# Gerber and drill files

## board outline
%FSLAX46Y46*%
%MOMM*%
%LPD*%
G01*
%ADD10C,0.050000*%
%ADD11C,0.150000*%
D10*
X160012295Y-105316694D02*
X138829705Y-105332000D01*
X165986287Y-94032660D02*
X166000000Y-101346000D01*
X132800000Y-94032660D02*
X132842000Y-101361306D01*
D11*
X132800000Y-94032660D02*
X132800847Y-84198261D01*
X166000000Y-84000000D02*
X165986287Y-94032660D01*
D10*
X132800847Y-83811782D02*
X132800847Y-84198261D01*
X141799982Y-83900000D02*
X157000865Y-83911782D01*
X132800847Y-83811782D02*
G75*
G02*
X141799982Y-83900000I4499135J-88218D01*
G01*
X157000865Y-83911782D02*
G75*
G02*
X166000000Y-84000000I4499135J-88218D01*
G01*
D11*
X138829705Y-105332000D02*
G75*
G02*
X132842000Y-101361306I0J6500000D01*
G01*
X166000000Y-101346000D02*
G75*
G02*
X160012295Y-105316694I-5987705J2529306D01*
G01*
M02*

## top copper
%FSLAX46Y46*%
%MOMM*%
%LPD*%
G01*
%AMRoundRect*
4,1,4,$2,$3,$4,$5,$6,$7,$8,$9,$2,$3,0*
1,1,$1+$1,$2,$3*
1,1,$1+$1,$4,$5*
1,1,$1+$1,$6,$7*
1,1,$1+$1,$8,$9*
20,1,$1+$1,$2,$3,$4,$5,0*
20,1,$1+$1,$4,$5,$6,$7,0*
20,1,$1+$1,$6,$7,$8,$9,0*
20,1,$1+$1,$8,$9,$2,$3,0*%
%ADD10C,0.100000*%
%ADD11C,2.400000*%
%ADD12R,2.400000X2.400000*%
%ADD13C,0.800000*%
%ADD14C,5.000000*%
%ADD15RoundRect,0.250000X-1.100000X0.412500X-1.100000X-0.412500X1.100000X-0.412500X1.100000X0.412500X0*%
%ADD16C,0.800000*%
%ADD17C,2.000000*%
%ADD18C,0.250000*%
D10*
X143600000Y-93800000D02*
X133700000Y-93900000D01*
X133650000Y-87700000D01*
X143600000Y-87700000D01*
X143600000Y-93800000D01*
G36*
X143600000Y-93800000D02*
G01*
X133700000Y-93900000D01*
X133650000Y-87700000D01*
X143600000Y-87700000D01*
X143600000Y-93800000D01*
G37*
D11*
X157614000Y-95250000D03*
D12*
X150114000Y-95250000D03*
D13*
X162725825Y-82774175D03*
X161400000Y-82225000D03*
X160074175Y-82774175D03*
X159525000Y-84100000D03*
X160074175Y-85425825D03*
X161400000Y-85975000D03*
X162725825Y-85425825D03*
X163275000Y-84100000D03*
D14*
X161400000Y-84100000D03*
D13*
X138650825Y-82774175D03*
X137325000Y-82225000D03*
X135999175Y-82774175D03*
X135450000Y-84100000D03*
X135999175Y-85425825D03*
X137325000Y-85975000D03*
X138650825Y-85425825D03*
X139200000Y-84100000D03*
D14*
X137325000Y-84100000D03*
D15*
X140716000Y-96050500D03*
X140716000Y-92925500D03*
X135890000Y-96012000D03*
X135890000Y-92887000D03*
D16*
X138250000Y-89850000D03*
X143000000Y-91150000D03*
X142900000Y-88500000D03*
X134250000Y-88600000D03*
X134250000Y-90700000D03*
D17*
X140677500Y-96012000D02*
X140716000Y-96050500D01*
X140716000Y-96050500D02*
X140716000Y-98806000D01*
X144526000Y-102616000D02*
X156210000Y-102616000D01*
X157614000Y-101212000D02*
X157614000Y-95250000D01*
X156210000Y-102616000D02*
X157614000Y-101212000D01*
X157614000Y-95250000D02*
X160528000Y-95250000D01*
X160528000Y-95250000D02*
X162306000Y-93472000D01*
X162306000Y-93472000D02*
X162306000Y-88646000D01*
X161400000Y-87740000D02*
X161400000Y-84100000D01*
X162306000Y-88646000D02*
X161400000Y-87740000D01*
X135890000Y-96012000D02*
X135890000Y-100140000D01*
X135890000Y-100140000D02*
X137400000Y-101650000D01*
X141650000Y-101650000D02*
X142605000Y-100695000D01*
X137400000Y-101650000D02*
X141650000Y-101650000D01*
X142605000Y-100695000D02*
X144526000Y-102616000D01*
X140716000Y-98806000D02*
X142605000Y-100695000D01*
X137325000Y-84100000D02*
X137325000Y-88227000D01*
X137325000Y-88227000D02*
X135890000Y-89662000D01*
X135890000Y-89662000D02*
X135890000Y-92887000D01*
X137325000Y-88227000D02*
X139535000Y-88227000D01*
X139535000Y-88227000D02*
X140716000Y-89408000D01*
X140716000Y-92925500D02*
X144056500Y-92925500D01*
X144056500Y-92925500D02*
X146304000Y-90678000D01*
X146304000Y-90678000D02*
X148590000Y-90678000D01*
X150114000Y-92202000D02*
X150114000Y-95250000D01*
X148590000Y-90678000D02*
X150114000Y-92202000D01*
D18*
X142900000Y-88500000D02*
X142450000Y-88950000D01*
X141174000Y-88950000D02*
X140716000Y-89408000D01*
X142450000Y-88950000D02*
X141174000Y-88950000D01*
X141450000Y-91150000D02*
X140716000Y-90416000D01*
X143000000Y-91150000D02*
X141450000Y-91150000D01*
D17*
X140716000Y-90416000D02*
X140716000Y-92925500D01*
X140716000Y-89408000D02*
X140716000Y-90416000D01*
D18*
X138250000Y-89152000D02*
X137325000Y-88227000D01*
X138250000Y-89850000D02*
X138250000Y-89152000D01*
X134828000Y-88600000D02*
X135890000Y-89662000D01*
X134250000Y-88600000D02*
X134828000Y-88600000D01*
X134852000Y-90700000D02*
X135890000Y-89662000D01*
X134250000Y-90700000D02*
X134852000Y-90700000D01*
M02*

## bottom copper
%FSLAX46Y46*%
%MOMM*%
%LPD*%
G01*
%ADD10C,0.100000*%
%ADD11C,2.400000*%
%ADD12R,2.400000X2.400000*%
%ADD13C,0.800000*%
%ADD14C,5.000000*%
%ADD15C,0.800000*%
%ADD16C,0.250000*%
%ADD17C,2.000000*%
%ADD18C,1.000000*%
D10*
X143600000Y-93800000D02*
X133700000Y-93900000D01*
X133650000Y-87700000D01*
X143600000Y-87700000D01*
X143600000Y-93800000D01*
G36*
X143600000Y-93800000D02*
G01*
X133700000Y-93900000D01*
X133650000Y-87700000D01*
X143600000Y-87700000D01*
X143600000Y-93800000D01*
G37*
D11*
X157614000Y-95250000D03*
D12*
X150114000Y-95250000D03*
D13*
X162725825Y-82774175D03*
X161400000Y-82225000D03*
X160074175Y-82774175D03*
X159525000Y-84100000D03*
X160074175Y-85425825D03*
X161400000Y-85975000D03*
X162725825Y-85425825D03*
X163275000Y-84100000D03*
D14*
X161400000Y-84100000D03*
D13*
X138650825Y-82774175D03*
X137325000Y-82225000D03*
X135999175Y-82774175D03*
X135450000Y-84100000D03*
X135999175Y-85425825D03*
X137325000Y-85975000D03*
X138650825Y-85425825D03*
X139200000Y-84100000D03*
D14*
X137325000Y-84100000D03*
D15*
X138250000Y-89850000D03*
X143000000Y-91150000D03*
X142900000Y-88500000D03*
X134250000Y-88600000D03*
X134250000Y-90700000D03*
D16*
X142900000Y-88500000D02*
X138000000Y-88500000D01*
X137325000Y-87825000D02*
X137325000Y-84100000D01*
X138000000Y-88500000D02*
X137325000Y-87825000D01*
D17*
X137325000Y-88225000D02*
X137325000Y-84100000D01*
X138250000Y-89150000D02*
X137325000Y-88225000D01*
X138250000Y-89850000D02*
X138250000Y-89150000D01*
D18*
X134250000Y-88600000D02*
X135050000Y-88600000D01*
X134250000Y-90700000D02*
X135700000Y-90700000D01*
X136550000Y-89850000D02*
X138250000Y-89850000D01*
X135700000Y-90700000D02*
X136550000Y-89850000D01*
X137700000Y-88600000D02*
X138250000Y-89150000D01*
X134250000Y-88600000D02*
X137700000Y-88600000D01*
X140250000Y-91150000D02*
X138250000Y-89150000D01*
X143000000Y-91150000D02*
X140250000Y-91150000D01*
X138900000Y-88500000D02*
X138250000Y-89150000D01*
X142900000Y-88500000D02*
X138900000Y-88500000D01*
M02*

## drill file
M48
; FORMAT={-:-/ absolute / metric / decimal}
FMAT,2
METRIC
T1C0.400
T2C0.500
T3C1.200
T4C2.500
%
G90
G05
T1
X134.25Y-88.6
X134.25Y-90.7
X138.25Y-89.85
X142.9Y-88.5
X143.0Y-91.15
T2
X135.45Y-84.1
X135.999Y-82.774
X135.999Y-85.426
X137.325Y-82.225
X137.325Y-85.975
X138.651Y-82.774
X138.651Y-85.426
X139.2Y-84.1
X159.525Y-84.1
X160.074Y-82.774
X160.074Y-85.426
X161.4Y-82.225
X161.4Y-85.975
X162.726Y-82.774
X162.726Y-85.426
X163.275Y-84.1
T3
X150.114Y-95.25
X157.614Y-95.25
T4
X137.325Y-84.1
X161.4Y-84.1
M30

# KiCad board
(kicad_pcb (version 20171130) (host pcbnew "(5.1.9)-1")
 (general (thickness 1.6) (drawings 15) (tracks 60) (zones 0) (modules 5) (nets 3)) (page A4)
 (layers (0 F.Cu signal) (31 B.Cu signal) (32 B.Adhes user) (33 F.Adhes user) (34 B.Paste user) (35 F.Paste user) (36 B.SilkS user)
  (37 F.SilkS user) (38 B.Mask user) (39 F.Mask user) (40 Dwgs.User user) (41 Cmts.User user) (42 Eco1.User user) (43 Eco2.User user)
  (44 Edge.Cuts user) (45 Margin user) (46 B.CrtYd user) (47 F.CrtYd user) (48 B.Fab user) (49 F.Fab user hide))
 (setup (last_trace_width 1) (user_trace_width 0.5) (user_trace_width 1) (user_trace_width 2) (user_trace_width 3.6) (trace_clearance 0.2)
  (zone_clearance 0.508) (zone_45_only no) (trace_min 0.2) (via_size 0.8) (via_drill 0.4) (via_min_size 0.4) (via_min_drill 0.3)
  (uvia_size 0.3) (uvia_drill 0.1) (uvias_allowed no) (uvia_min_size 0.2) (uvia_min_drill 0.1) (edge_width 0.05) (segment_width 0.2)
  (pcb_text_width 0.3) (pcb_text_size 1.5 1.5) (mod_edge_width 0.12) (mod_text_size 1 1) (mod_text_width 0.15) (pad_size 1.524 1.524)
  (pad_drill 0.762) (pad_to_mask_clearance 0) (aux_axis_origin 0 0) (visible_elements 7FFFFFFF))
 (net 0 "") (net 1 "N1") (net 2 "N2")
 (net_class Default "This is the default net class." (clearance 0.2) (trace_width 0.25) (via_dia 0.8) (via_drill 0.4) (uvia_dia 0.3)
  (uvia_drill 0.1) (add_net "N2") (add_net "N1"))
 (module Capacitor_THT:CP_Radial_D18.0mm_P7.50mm (layer F.Cu) (at 150.114 95.25)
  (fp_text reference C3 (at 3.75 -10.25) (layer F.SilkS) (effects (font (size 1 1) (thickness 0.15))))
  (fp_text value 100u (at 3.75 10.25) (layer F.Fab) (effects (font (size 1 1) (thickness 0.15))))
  (pad 2 thru_hole circle (at 7.5 0) (size 2.4 2.4) (drill 1.2) (layers *.Cu *.Mask) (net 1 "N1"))
  (pad 1 thru_hole rect (at 0 0) (size 2.4 2.4) (drill 1.2) (layers *.Cu *.Mask) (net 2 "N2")))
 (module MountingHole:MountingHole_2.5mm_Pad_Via (layer F.Cu) (at 161.4 84.1)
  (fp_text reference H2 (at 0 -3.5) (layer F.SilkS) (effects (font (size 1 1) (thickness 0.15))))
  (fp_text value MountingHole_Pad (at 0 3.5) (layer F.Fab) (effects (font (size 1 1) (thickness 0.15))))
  (pad 1 thru_hole circle (at 1.325825 -1.325825) (size 0.8 0.8) (drill 0.5) (layers *.Cu *.Mask) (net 1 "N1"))
  (pad 1 thru_hole circle (at 0 -1.875) (size 0.8 0.8) (drill 0.5) (layers *.Cu *.Mask) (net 1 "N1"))
  (pad 1 thru_hole circle (at -1.325825 -1.325825) (size 0.8 0.8) (drill 0.5) (layers *.Cu *.Mask) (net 1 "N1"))
  (pad 1 thru_hole circle (at -1.875 0) (size 0.8 0.8) (drill 0.5) (layers *.Cu *.Mask) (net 1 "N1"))
  (pad 1 thru_hole circle (at -1.325825 1.325825) (size 0.8 0.8) (drill 0.5) (layers *.Cu *.Mask) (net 1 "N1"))
  (pad 1 thru_hole circle (at 0 1.875) (size 0.8 0.8) (drill 0.5) (layers *.Cu *.Mask) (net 1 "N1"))
  (pad 1 thru_hole circle (at 1.325825 1.325825) (size 0.8 0.8) (drill 0.5) (layers *.Cu *.Mask) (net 1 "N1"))
  (pad 1 thru_hole circle (at 1.875 0) (size 0.8 0.8) (drill 0.5) (layers *.Cu *.Mask) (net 1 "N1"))
  (pad 1 thru_hole circle (at 0 0) (size 5 5) (drill 2.5) (layers *.Cu *.Mask) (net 1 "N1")))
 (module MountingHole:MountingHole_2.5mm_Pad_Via (layer F.Cu) (at 137.325 84.1)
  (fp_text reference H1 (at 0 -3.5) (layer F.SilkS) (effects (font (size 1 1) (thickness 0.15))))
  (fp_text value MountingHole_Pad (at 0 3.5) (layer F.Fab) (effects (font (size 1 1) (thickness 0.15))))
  (pad 1 thru_hole circle (at 1.325825 -1.325825) (size 0.8 0.8) (drill 0.5) (layers *.Cu *.Mask) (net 2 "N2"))
  (pad 1 thru_hole circle (at 0 -1.875) (size 0.8 0.8) (drill 0.5) (layers *.Cu *.Mask) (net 2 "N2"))
  (pad 1 thru_hole circle (at -1.325825 -1.325825) (size 0.8 0.8) (drill 0.5) (layers *.Cu *.Mask) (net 2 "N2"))
  (pad 1 thru_hole circle (at -1.875 0) (size 0.8 0.8) (drill 0.5) (layers *.Cu *.Mask) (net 2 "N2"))
  (pad 1 thru_hole circle (at -1.325825 1.325825) (size 0.8 0.8) (drill 0.5) (layers *.Cu *.Mask) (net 2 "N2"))
  (pad 1 thru_hole circle (at 0 1.875) (size 0.8 0.8) (drill 0.5) (layers *.Cu *.Mask) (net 2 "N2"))
  (pad 1 thru_hole circle (at 1.325825 1.325825) (size 0.8 0.8) (drill 0.5) (layers *.Cu *.Mask) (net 2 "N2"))
  (pad 1 thru_hole circle (at 1.875 0) (size 0.8 0.8) (drill 0.5) (layers *.Cu *.Mask) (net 2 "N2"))
  (pad 1 thru_hole circle (at 0 0) (size 5 5) (drill 2.5) (layers *.Cu *.Mask) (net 2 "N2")))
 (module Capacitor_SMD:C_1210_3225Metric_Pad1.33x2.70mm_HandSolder (layer F.Cu) (at 140.716 94.488 270)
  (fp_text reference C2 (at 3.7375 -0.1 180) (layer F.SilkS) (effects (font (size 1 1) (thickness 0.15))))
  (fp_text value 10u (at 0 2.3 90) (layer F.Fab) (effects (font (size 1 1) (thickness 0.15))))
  (pad 2 smd roundrect (at 1.5625 0 270) (size 1.325 2.7) (layers F.Cu F.Paste F.Mask) (roundrect_rratio 0.188679) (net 1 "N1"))
  (pad 1 smd roundrect (at -1.5625 0 270) (size 1.325 2.7) (layers F.Cu F.Paste F.Mask) (roundrect_rratio 0.188679) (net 2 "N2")))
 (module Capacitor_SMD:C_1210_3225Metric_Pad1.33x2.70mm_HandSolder (layer F.Cu) (at 135.89 94.4495 270)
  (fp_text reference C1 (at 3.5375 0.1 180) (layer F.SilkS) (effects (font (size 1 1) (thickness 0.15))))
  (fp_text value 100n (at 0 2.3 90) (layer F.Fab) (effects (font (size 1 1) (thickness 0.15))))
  (pad 2 smd roundrect (at 1.5625 0 270) (size 1.325 2.7) (layers F.Cu F.Paste F.Mask) (roundrect_rratio 0.188679) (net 1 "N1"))
  (pad 1 smd roundrect (at -1.5625 0 270) (size 1.325 2.7) (layers F.Cu F.Paste F.Mask) (roundrect_rratio 0.188679) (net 2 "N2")))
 (gr_poly (pts (xy 143.6 93.8) (xy 133.7 93.9) (xy 133.65 87.7) (xy 143.6 87.7)) (layer B.Cu) (width 0.1))
 (gr_poly (pts (xy 143.6 93.8) (xy 133.7 93.9) (xy 133.65 87.7) (xy 143.6 87.7)) (layer F.Cu) (width 0.1))
 (gr_line (start 160.012295 105.316694) (end 138.829705 105.332) (layer Edge.Cuts) (width 0.05))
 (gr_line (start 165.986287 94.03266) (end 166 101.346) (layer Edge.Cuts) (width 0.05))
 (gr_line (start 132.8 94.03266) (end 132.842 101.361306) (layer Edge.Cuts) (width 0.05))
 (gr_line (start 132.8 94.03266) (end 132.800847 84.198261) (layer Edge.Cuts) (width 0.15))
 (gr_line (start 166 84) (end 165.986287 94.03266) (layer Edge.Cuts) (width 0.15))
 (gr_line (start 132.800847 83.811782) (end 132.800847 84.198261) (layer Edge.Cuts) (width 0.05))
 (gr_line (start 141.799982 83.9) (end 157.000865 83.911782) (layer Edge.Cuts) (width 0.05))
 (gr_arc (start 137.299982 83.9) (end 141.799982 83.9) (angle -178.8766973) (layer Edge.Cuts) (width 0.05))
 (gr_arc (start 161.5 84) (end 166 84) (angle -178.8766973) (layer Edge.Cuts) (width 0.05))
 (gr_arc (start 138.829705 98.832) (end 138.829705 105.332) (angle 67.1) (layer Edge.Cuts) (width 0.15))
 (gr_arc (start 160.012295 98.816694) (end 160.012295 105.316694) (angle -67.1) (layer Edge.Cuts) (width 0.15))
 (via (at 138.25 89.85) (size 0.8) (drill 0.4) (layers F.Cu B.Cu) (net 2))
 (via (at 143 91.15) (size 0.8) (drill 0.4) (layers F.Cu B.Cu) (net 2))
 (via (at 142.9 88.5) (size 0.8) (drill 0.4) (layers F.Cu B.Cu) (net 2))
 (via (at 134.25 88.6) (size 0.8) (drill 0.4) (layers F.Cu B.Cu) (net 2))
 (via (at 134.25 90.7) (size 0.8) (drill 0.4) (layers F.Cu B.Cu) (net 2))
 (segment (start 140.6775 96.012) (end 140.716 96.0505) (width 2) (layer F.Cu) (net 1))
 (segment (start 140.716 96.0505) (end 140.716 98.806) (width 2) (layer F.Cu) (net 1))
 (segment (start 144.526 102.616) (end 156.21 102.616) (width 2) (layer F.Cu) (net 1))
 (segment (start 157.614 101.212) (end 157.614 95.25) (width 2) (layer F.Cu) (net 1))
 (segment (start 156.21 102.616) (end 157.614 101.212) (width 2) (layer F.Cu) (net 1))
 (segment (start 157.614 95.25) (end 160.528 95.25) (width 2) (layer F.Cu) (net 1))
 (segment (start 160.528 95.25) (end 162.306 93.472) (width 2) (layer F.Cu) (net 1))
 (segment (start 162.306 93.472) (end 162.306 88.646) (width 2) (layer F.Cu) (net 1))
 (segment (start 161.4 87.74) (end 161.4 84.1) (width 2) (layer F.Cu) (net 1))
 (segment (start 162.306 88.646) (end 161.4 87.74) (width 2) (layer F.Cu) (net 1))
 (segment (start 135.89 96.012) (end 135.89 100.14) (width 2) (layer F.Cu) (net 1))
 (segment (start 135.89 100.14) (end 137.4 101.65) (width 2) (layer F.Cu) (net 1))
 (segment (start 141.65 101.65) (end 142.605 100.695) (width 2) (layer F.Cu) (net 1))
 (segment (start 137.4 101.65) (end 141.65 101.65) (width 2) (layer F.Cu) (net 1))
 (segment (start 142.605 100.695) (end 144.526 102.616) (width 2) (layer F.Cu) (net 1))
 (segment (start 140.716 98.806) (end 142.605 100.695) (width 2) (layer F.Cu) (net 1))
 (segment (start 137.325 84.1) (end 137.325 88.227) (width 2) (layer F.Cu) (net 2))
 (segment (start 137.325 88.227) (end 135.89 89.662) (width 2) (layer F.Cu) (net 2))
 (segment (start 135.89 89.662) (end 135.89 92.887) (width 2) (layer F.Cu) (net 2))
 (segment (start 137.325 88.227) (end 139.535 88.227) (width 2) (layer F.Cu) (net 2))
 (segment (start 139.535 88.227) (end 140.716 89.408) (width 2) (layer F.Cu) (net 2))
 (segment (start 140.716 92.9255) (end 144.0565 92.9255) (width 2) (layer F.Cu) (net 2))
 (segment (start 144.0565 92.9255) (end 146.304 90.678) (width 2) (layer F.Cu) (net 2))
 (segment (start 146.304 90.678) (end 148.59 90.678) (width 2) (layer F.Cu) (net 2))
 (segment (start 150.114 92.202) (end 150.114 95.25) (width 2) (layer F.Cu) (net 2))
 (segment (start 148.59 90.678) (end 150.114 92.202) (width 2) (layer F.Cu) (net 2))
 (segment (start 142.9 88.5) (end 142.45 88.95) (width 0.25) (layer F.Cu) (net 2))
 (segment (start 141.174 88.95) (end 140.716 89.408) (width 0.25) (layer F.Cu) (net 2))
 (segment (start 142.45 88.95) (end 141.174 88.95) (width 0.25) (layer F.Cu) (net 2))
 (segment (start 141.45 91.15) (end 140.716 90.416) (width 0.25) (layer F.Cu) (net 2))
 (segment (start 143 91.15) (end 141.45 91.15) (width 0.25) (layer F.Cu) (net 2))
 (segment (start 140.716 90.416) (end 140.716 92.9255) (width 2) (layer F.Cu) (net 2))
 (segment (start 140.716 89.408) (end 140.716 90.416) (width 2) (layer F.Cu) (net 2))
 (segment (start 138.25 89.152) (end 137.325 88.227) (width 0.25) (layer F.Cu) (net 2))
 (segment (start 138.25 89.85) (end 138.25 89.152) (width 0.25) (layer F.Cu) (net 2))
 (segment (start 134.828 88.6) (end 135.89 89.662) (width 0.25) (layer F.Cu) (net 2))
 (segment (start 134.25 88.6) (end 134.828 88.6) (width 0.25) (layer F.Cu) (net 2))
 (segment (start 134.852 90.7) (end 135.89 89.662) (width 0.25) (layer F.Cu) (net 2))
 (segment (start 134.25 90.7) (end 134.852 90.7) (width 0.25) (layer F.Cu) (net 2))
 (segment (start 142.9 88.5) (end 138 88.5) (width 0.25) (layer B.Cu) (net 2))
 (segment (start 137.325 87.825) (end 137.325 84.1) (width 0.25) (layer B.Cu) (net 2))
 (segment (start 138 88.5) (end 137.325 87.825) (width 0.25) (layer B.Cu) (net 2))
 (segment (start 137.325 88.225) (end 137.325 84.1) (width 2) (layer B.Cu) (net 2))
 (segment (start 138.25 89.15) (end 137.325 88.225) (width 2) (layer B.Cu) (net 2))
 (segment (start 138.25 89.85) (end 138.25 89.15) (width 2) (layer B.Cu) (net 2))
 (segment (start 134.25 88.6) (end 135.05 88.6) (width 1) (layer B.Cu) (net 2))
 (segment (start 134.25 90.7) (end 135.7 90.7) (width 1) (layer B.Cu) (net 2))
 (segment (start 136.55 89.85) (end 138.25 89.85) (width 1) (layer B.Cu) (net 2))
 (segment (start 135.7 90.7) (end 136.55 89.85) (width 1) (layer B.Cu) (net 2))
 (segment (start 137.7 88.6) (end 138.25 89.15) (width 1) (layer B.Cu) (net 2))
 (segment (start 134.25 88.6) (end 137.7 88.6) (width 1) (layer B.Cu) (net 2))
 (segment (start 140.25 91.15) (end 138.25 89.15) (width 1) (layer B.Cu) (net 2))
 (segment (start 143 91.15) (end 140.25 91.15) (width 1) (layer B.Cu) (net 2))
 (segment (start 138.9 88.5) (end 138.25 89.15) (width 1) (layer B.Cu) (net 2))
 (segment (start 142.9 88.5) (end 138.9 88.5) (width 1) (layer B.Cu) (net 2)))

